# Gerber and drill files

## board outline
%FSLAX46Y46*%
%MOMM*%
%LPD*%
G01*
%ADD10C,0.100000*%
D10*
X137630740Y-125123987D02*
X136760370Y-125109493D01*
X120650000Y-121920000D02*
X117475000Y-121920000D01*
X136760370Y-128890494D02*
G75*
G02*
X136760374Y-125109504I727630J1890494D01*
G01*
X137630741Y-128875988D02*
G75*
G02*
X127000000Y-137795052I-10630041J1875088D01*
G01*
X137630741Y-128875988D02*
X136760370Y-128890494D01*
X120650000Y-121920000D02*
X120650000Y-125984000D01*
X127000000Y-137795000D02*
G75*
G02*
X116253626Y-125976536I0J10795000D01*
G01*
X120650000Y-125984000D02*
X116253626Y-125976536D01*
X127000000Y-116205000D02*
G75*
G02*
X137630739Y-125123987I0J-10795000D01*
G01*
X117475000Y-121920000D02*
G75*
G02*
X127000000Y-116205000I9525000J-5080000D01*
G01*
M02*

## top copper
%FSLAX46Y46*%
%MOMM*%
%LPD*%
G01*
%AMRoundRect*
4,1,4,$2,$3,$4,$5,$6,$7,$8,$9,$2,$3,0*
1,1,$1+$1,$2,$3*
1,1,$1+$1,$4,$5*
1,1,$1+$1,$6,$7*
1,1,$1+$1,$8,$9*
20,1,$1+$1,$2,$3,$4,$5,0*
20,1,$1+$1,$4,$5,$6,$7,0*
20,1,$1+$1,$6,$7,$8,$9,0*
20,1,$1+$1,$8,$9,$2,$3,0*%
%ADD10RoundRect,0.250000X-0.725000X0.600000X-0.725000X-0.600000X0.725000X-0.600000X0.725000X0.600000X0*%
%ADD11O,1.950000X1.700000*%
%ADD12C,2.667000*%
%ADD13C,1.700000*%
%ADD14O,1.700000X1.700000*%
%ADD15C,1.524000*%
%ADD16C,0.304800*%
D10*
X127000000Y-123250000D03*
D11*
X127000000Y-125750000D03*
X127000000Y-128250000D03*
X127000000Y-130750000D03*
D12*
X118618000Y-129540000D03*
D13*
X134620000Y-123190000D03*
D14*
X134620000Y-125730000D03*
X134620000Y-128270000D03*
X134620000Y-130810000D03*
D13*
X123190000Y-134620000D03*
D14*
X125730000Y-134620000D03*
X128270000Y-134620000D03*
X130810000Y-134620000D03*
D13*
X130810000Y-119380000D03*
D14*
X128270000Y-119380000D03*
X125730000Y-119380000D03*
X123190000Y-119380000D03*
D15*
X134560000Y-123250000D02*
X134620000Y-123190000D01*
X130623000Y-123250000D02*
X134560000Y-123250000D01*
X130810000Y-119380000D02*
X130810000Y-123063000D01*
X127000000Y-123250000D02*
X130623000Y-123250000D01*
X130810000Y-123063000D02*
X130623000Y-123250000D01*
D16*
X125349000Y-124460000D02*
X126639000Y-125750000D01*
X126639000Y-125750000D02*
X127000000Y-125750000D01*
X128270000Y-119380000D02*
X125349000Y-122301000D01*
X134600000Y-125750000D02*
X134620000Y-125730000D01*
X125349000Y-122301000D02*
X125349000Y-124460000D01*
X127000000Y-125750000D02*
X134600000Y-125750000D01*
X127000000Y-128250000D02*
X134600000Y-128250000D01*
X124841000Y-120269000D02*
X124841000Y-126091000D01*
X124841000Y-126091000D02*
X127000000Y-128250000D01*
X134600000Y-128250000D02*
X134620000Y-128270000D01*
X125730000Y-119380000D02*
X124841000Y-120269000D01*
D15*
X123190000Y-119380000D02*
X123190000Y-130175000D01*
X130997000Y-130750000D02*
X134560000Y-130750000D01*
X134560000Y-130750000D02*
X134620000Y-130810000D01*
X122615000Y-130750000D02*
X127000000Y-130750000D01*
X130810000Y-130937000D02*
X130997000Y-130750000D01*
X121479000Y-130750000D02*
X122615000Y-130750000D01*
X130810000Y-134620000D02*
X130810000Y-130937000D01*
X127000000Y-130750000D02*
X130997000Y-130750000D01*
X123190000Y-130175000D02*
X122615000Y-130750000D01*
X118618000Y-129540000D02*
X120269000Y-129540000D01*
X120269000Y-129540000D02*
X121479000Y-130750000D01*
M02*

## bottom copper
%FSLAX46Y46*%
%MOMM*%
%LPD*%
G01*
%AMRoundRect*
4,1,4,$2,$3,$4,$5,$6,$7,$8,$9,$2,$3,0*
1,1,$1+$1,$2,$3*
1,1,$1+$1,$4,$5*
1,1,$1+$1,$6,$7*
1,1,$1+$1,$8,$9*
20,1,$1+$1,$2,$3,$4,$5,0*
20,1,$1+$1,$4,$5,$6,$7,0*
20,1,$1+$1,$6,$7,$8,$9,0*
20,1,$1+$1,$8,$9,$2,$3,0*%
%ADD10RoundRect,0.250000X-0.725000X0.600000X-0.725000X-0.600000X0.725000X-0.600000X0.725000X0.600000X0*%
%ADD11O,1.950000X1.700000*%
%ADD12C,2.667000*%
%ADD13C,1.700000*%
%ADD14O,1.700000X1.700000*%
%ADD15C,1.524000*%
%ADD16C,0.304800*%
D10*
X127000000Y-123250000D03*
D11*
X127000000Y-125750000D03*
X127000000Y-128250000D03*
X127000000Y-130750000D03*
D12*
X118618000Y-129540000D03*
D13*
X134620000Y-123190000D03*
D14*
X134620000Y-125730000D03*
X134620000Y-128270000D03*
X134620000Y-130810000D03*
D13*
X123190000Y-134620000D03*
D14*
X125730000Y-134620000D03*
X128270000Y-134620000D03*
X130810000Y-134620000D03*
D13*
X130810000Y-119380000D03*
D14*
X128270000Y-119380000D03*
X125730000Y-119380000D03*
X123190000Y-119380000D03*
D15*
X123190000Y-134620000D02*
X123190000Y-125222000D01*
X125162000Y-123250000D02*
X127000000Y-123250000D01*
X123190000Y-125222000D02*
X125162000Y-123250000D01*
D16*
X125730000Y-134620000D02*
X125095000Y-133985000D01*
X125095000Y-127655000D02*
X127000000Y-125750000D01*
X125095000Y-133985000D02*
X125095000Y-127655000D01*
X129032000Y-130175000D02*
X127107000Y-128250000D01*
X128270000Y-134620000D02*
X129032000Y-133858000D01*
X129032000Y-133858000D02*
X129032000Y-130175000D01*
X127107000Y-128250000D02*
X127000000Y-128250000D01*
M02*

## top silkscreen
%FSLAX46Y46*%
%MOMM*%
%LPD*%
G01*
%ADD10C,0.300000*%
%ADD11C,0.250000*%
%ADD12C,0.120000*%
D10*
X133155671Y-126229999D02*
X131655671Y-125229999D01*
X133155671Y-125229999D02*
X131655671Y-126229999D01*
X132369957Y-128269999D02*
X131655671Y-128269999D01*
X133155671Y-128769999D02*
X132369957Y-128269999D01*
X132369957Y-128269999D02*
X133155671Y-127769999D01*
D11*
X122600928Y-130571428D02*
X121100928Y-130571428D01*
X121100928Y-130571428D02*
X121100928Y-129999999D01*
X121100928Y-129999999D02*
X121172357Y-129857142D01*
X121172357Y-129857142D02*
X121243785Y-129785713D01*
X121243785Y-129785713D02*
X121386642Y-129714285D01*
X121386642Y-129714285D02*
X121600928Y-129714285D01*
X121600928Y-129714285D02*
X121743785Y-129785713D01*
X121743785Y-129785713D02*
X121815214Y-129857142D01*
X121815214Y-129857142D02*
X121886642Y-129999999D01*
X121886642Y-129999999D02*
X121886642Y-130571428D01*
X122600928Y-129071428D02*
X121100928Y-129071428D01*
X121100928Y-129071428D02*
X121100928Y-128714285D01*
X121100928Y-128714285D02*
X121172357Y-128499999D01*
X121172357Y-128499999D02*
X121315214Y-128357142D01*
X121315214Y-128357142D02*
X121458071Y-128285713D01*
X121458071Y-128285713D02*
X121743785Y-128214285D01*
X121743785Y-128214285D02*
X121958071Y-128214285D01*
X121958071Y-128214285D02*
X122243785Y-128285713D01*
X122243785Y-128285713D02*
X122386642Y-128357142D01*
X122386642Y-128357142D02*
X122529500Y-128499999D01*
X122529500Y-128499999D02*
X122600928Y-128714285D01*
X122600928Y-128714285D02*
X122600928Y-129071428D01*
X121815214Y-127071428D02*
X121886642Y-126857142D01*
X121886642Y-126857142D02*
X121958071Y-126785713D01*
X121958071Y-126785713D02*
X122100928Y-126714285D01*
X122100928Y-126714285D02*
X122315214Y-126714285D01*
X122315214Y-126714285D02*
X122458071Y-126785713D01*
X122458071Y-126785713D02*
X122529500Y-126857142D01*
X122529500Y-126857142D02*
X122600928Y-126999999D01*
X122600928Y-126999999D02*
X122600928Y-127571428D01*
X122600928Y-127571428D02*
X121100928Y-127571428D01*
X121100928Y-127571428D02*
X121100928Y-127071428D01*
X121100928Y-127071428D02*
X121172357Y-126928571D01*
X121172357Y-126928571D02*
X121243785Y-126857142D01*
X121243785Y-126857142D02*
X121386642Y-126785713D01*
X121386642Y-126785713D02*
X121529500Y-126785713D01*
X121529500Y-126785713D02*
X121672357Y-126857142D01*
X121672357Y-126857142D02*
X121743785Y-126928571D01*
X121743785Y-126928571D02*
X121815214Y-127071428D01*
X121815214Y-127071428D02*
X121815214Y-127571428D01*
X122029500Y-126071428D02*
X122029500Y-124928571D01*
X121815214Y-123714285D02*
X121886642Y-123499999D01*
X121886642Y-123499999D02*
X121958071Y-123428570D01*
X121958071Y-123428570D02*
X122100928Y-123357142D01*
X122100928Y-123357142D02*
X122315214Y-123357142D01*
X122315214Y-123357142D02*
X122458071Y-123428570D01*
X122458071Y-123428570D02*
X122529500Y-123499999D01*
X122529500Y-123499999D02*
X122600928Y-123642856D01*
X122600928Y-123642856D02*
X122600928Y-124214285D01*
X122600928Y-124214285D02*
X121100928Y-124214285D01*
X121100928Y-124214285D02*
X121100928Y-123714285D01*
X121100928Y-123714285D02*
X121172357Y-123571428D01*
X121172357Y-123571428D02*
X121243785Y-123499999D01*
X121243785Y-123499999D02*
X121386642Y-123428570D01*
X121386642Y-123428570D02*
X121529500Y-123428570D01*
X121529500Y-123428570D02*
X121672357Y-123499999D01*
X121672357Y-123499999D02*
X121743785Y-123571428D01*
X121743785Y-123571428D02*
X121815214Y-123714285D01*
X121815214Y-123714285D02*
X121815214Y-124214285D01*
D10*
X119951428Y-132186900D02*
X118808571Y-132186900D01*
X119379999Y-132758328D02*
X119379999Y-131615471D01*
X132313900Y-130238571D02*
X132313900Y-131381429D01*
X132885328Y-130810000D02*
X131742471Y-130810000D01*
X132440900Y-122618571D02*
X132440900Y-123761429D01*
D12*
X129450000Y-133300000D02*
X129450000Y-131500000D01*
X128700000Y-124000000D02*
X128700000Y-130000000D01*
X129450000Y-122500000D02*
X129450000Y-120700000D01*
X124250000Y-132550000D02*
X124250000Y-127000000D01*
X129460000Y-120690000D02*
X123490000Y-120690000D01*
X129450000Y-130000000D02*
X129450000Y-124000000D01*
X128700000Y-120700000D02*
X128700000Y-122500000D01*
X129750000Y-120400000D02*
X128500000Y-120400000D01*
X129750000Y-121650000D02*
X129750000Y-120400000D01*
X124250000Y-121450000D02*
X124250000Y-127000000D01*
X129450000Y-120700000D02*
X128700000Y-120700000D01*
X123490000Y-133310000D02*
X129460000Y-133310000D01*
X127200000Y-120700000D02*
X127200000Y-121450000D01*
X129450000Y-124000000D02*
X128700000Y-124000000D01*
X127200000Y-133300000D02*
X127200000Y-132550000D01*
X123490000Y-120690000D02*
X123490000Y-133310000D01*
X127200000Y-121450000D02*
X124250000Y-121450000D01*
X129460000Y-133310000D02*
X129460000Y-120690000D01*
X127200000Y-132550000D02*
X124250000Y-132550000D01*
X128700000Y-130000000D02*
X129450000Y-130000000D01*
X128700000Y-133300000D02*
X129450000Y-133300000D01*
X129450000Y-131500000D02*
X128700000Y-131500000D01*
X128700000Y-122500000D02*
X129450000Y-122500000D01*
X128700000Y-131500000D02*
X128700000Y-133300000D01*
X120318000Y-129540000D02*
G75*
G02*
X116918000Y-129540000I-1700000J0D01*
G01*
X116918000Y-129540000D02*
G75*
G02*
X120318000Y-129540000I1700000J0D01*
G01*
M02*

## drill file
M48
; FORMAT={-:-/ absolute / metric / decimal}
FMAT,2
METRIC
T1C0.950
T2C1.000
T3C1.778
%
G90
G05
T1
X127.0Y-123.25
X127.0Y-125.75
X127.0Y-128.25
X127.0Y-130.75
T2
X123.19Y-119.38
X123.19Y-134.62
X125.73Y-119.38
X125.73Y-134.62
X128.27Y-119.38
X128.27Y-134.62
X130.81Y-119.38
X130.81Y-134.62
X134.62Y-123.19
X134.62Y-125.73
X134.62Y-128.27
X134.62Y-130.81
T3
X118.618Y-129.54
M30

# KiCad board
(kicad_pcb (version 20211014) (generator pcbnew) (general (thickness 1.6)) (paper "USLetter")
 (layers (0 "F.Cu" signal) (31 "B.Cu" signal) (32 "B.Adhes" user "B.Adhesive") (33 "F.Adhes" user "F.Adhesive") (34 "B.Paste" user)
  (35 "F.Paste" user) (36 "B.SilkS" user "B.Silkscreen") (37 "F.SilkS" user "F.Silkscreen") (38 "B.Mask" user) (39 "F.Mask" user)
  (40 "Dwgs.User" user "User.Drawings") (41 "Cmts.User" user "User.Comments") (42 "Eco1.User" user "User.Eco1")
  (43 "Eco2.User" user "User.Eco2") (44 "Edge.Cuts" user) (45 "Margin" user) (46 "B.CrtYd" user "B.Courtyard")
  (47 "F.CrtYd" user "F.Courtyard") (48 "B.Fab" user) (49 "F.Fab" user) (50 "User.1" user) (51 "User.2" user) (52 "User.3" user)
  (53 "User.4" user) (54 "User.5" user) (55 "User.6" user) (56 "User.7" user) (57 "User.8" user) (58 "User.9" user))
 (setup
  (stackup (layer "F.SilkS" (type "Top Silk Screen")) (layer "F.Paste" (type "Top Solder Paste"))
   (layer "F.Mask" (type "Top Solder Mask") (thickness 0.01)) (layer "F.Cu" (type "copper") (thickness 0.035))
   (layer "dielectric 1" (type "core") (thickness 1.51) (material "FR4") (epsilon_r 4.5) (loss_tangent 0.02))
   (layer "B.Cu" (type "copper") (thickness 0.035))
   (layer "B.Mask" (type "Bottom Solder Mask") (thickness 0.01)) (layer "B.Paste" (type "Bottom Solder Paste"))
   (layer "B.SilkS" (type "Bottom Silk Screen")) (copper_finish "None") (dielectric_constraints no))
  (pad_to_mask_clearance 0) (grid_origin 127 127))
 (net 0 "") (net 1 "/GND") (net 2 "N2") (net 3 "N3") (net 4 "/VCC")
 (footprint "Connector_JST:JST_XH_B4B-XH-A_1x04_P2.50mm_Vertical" (layer "F.Cu") (at 127 123.25 -90)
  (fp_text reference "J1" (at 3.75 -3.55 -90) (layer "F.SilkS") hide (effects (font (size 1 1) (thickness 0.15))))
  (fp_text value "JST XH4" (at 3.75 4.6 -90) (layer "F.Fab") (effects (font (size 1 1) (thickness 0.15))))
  (fp_line (start 10.05 -2.45) (end 8.25 -2.45) (layer "F.SilkS") (width 0.12))
  (fp_line (start 0.75 -1.7) (end 6.75 -1.7) (layer "F.SilkS") (width 0.12))
  (fp_line (start -0.75 -2.45) (end -2.55 -2.45) (layer "F.SilkS") (width 0.12))
  (fp_line (start 9.3 2.75) (end 3.75 2.75) (layer "F.SilkS") (width 0.12))
  (fp_line (start -2.56 -2.46) (end -2.56 3.51) (layer "F.SilkS") (width 0.12))
  (fp_line (start 6.75 -2.45) (end 0.75 -2.45) (layer "F.SilkS") (width 0.12))
  (fp_line (start -2.55 -1.7) (end -0.75 -1.7) (layer "F.SilkS") (width 0.12))
  (fp_line (start -2.85 -2.75) (end -2.85 -1.5) (layer "F.SilkS") (width 0.12))
  (fp_line (start -1.6 -2.75) (end -2.85 -2.75) (layer "F.SilkS") (width 0.12))
  (fp_line (start -1.8 2.75) (end 3.75 2.75) (layer "F.SilkS") (width 0.12))
  (fp_line (start -2.55 -2.45) (end -2.55 -1.7) (layer "F.SilkS") (width 0.12))
  (fp_line (start 10.06 3.51) (end 10.06 -2.46) (layer "F.SilkS") (width 0.12))
  (fp_line (start -2.55 -0.2) (end -1.8 -0.2) (layer "F.SilkS") (width 0.12))
  (fp_line (start 0.75 -2.45) (end 0.75 -1.7) (layer "F.SilkS") (width 0.12))
  (fp_line (start 10.05 -0.2) (end 9.3 -0.2) (layer "F.SilkS") (width 0.12))
  (fp_line (start -2.56 3.51) (end 10.06 3.51) (layer "F.SilkS") (width 0.12))
  (fp_line (start -1.8 -0.2) (end -1.8 2.75) (layer "F.SilkS") (width 0.12))
  (fp_line (start 10.06 -2.46) (end -2.56 -2.46) (layer "F.SilkS") (width 0.12))
  (fp_line (start 9.3 -0.2) (end 9.3 2.75) (layer "F.SilkS") (width 0.12))
  (fp_line (start 6.75 -1.7) (end 6.75 -2.45) (layer "F.SilkS") (width 0.12))
  (fp_line (start 10.05 -1.7) (end 10.05 -2.45) (layer "F.SilkS") (width 0.12))
  (fp_line (start 8.25 -2.45) (end 8.25 -1.7) (layer "F.SilkS") (width 0.12))
  (fp_line (start -0.75 -1.7) (end -0.75 -2.45) (layer "F.SilkS") (width 0.12))
  (fp_line (start 8.25 -1.7) (end 10.05 -1.7) (layer "F.SilkS") (width 0.12))
  (pad "1" thru_hole roundrect (at 0 0 270) (size 1.7 1.95) (drill 0.95) (layers *.Cu *.Mask) (roundrect_rratio 0.1470588235) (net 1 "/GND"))
  (pad "2" thru_hole oval (at 2.5 0 270) (size 1.7 1.95) (drill 0.95) (layers *.Cu *.Mask) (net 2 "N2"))
  (pad "3" thru_hole oval (at 5 0 270) (size 1.7 1.95) (drill 0.95) (layers *.Cu *.Mask) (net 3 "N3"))
  (pad "4" thru_hole oval (at 7.5 0 270) (size 1.7 1.95) (drill 0.95) (layers *.Cu *.Mask) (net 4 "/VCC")))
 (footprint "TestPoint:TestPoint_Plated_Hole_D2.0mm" (layer "F.Cu") (at 118.618 129.54)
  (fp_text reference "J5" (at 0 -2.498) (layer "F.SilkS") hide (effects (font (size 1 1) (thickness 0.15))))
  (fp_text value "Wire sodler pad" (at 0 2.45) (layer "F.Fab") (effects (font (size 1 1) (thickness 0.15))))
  (fp_circle (center 0 0) (end 0 -1.7) (layer "F.SilkS") (width 0.12) (fill none))
  (pad "1" thru_hole circle (at 0 0) (size 2.667 2.667) (drill 1.778) (layers *.Cu *.Mask) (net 4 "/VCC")))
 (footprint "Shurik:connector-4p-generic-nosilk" (layer "F.Cu") (at 134.62 123.19)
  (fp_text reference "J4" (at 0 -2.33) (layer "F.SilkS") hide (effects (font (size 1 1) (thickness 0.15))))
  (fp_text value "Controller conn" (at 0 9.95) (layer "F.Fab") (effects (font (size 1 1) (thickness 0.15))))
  (pad "1" thru_hole circle (at 0 0) (size 1.7 1.7) (drill 1) (layers *.Cu *.Mask) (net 1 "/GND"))
  (pad "2" thru_hole oval (at 0 2.54) (size 1.7 1.7) (drill 1) (layers *.Cu *.Mask) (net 2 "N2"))
  (pad "3" thru_hole oval (at 0 5.08) (size 1.7 1.7) (drill 1) (layers *.Cu *.Mask) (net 3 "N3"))
  (pad "4" thru_hole oval (at 0 7.62) (size 1.7 1.7) (drill 1) (layers *.Cu *.Mask) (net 4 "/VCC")))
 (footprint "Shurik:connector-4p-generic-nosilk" (layer "F.Cu") (at 123.19 134.62 90)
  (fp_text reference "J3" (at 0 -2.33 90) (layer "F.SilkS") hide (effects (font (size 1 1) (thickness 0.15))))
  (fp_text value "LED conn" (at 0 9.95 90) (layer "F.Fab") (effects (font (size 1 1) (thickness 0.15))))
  (pad "1" thru_hole circle (at 0 0 90) (size 1.7 1.7) (drill 1) (layers *.Cu *.Mask) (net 1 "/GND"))
  (pad "2" thru_hole oval (at 0 2.54 90) (size 1.7 1.7) (drill 1) (layers *.Cu *.Mask) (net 2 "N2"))
  (pad "3" thru_hole oval (at 0 5.08 90) (size 1.7 1.7) (drill 1) (layers *.Cu *.Mask) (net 3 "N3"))
  (pad "4" thru_hole oval (at 0 7.62 90) (size 1.7 1.7) (drill 1) (layers *.Cu *.Mask) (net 4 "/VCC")))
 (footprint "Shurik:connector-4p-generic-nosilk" (layer "F.Cu") (at 130.81 119.38 -90)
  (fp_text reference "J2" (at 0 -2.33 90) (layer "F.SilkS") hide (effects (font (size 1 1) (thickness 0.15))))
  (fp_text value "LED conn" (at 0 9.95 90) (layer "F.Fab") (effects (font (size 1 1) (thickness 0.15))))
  (pad "1" thru_hole circle (at 0 0 270) (size 1.7 1.7) (drill 1) (layers *.Cu *.Mask) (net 1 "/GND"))
  (pad "2" thru_hole oval (at 0 2.54 270) (size 1.7 1.7) (drill 1) (layers *.Cu *.Mask) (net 2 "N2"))
  (pad "3" thru_hole oval (at 0 5.08 270) (size 1.7 1.7) (drill 1) (layers *.Cu *.Mask) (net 3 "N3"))
  (pad "4" thru_hole oval (at 0 7.62 270) (size 1.7 1.7) (drill 1) (layers *.Cu *.Mask) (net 4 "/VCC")))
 (gr_line (start 137.63074 125.123987) (end 136.76037 125.109493) (layer "Edge.Cuts") (width 0.1))
 (gr_line (start 120.65 121.92) (end 117.475 121.92) (layer "Edge.Cuts") (width 0.1))
 (gr_arc (start 136.76037 128.890494) (mid 135.462276 126.999993) (end 136.76037 125.109493) (layer "Edge.Cuts") (width 0.1))
 (gr_arc (start 137.630741 128.875988) (mid 133.938498 135.27013) (end 127 137.795) (layer "Edge.Cuts") (width 0.1))
 (gr_line (start 137.630741 128.875988) (end 136.76037 128.890494) (layer "Edge.Cuts") (width 0.1))
 (gr_line (start 120.65 121.92) (end 120.65 125.984) (layer "Edge.Cuts") (width 0.1))
 (gr_arc (start 127 137.795) (mid 119.013129 134.262356) (end 116.253626 125.976536) (layer "Edge.Cuts") (width 0.1))
 (gr_line (start 120.65 125.984) (end 116.253626 125.976536) (layer "Edge.Cuts") (width 0.1))
 (gr_arc (start 127 116.205) (mid 133.93832 118.730063) (end 137.63074 125.123987) (layer "Edge.Cuts") (width 0.1))
 (gr_arc (start 117.475 121.92) (mid 121.446017 117.743361) (end 127 116.205) (layer "Edge.Cuts") (width 0.1))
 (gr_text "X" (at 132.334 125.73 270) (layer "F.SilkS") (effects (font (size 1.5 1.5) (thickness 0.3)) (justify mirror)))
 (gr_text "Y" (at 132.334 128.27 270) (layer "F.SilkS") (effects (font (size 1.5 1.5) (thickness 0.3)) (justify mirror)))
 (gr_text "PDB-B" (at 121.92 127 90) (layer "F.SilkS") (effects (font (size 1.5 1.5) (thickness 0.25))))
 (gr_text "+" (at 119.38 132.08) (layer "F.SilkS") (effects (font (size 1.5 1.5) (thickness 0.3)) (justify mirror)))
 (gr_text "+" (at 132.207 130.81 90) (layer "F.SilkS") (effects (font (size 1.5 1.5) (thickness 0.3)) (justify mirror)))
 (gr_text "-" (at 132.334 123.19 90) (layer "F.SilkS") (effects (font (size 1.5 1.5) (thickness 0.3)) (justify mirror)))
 (segment (start 134.56 123.25) (end 134.62 123.19) (width 1.524) (layer "F.Cu") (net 1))
 (segment (start 130.623 123.25) (end 134.56 123.25) (width 1.524) (layer "F.Cu") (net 1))
 (segment (start 130.81 119.38) (end 130.81 123.063) (width 1.524) (layer "F.Cu") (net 1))
 (segment (start 127 123.25) (end 130.623 123.25) (width 1.524) (layer "F.Cu") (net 1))
 (segment (start 130.81 123.063) (end 130.623 123.25) (width 1.524) (layer "F.Cu") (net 1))
 (segment (start 123.19 134.62) (end 123.19 125.222) (width 1.524) (layer "B.Cu") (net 1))
 (segment (start 125.162 123.25) (end 127 123.25) (width 1.524) (layer "B.Cu") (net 1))
 (segment (start 123.19 125.222) (end 125.162 123.25) (width 1.524) (layer "B.Cu") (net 1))
 (segment (start 125.349 124.46) (end 126.639 125.75) (width 0.3048) (layer "F.Cu") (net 2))
 (segment (start 126.639 125.75) (end 127 125.75) (width 0.3048) (layer "F.Cu") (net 2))
 (segment (start 128.27 119.38) (end 125.349 122.301) (width 0.3048) (layer "F.Cu") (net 2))
 (segment (start 134.6 125.75) (end 134.62 125.73) (width 0.3048) (layer "F.Cu") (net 2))
 (segment (start 125.349 122.301) (end 125.349 124.46) (width 0.3048) (layer "F.Cu") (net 2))
 (segment (start 127 125.75) (end 134.6 125.75) (width 0.3048) (layer "F.Cu") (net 2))
 (segment (start 125.73 134.62) (end 125.095 133.985) (width 0.3048) (layer "B.Cu") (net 2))
 (segment (start 125.095 127.655) (end 127 125.75) (width 0.3048) (layer "B.Cu") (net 2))
 (segment (start 125.095 133.985) (end 125.095 127.655) (width 0.3048) (layer "B.Cu") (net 2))
 (segment (start 127 128.25) (end 134.6 128.25) (width 0.3048) (layer "F.Cu") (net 3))
 (segment (start 124.841 120.269) (end 124.841 126.091) (width 0.3048) (layer "F.Cu") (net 3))
 (segment (start 124.841 126.091) (end 127 128.25) (width 0.3048) (layer "F.Cu") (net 3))
 (segment (start 134.6 128.25) (end 134.62 128.27) (width 0.3048) (layer "F.Cu") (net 3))
 (segment (start 125.73 119.38) (end 124.841 120.269) (width 0.3048) (layer "F.Cu") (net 3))
 (segment (start 129.032 130.175) (end 127.107 128.25) (width 0.3048) (layer "B.Cu") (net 3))
 (segment (start 128.27 134.62) (end 129.032 133.858) (width 0.3048) (layer "B.Cu") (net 3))
 (segment (start 129.032 133.858) (end 129.032 130.175) (width 0.3048) (layer "B.Cu") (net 3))
 (segment (start 127.107 128.25) (end 127 128.25) (width 0.3048) (layer "B.Cu") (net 3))
 (segment (start 123.19 119.38) (end 123.19 130.175) (width 1.524) (layer "F.Cu") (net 4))
 (segment (start 130.997 130.75) (end 134.56 130.75) (width 1.524) (layer "F.Cu") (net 4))
 (segment (start 134.56 130.75) (end 134.62 130.81) (width 1.524) (layer "F.Cu") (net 4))
 (segment (start 122.615 130.75) (end 127 130.75) (width 1.524) (layer "F.Cu") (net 4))
 (segment (start 130.81 130.937) (end 130.997 130.75) (width 1.524) (layer "F.Cu") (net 4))
 (segment (start 121.479 130.75) (end 122.615 130.75) (width 1.524) (layer "F.Cu") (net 4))
 (segment (start 130.81 134.62) (end 130.81 130.937) (width 1.524) (layer "F.Cu") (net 4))
 (segment (start 127 130.75) (end 130.997 130.75) (width 1.524) (layer "F.Cu") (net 4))
 (segment (start 123.19 130.175) (end 122.615 130.75) (width 1.524) (layer "F.Cu") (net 4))
 (segment (start 118.618 129.54) (end 120.269 129.54) (width 1.524) (layer "F.Cu") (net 4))
 (segment (start 120.269 129.54) (end 121.479 130.75) (width 1.524) (layer "F.Cu") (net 4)))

